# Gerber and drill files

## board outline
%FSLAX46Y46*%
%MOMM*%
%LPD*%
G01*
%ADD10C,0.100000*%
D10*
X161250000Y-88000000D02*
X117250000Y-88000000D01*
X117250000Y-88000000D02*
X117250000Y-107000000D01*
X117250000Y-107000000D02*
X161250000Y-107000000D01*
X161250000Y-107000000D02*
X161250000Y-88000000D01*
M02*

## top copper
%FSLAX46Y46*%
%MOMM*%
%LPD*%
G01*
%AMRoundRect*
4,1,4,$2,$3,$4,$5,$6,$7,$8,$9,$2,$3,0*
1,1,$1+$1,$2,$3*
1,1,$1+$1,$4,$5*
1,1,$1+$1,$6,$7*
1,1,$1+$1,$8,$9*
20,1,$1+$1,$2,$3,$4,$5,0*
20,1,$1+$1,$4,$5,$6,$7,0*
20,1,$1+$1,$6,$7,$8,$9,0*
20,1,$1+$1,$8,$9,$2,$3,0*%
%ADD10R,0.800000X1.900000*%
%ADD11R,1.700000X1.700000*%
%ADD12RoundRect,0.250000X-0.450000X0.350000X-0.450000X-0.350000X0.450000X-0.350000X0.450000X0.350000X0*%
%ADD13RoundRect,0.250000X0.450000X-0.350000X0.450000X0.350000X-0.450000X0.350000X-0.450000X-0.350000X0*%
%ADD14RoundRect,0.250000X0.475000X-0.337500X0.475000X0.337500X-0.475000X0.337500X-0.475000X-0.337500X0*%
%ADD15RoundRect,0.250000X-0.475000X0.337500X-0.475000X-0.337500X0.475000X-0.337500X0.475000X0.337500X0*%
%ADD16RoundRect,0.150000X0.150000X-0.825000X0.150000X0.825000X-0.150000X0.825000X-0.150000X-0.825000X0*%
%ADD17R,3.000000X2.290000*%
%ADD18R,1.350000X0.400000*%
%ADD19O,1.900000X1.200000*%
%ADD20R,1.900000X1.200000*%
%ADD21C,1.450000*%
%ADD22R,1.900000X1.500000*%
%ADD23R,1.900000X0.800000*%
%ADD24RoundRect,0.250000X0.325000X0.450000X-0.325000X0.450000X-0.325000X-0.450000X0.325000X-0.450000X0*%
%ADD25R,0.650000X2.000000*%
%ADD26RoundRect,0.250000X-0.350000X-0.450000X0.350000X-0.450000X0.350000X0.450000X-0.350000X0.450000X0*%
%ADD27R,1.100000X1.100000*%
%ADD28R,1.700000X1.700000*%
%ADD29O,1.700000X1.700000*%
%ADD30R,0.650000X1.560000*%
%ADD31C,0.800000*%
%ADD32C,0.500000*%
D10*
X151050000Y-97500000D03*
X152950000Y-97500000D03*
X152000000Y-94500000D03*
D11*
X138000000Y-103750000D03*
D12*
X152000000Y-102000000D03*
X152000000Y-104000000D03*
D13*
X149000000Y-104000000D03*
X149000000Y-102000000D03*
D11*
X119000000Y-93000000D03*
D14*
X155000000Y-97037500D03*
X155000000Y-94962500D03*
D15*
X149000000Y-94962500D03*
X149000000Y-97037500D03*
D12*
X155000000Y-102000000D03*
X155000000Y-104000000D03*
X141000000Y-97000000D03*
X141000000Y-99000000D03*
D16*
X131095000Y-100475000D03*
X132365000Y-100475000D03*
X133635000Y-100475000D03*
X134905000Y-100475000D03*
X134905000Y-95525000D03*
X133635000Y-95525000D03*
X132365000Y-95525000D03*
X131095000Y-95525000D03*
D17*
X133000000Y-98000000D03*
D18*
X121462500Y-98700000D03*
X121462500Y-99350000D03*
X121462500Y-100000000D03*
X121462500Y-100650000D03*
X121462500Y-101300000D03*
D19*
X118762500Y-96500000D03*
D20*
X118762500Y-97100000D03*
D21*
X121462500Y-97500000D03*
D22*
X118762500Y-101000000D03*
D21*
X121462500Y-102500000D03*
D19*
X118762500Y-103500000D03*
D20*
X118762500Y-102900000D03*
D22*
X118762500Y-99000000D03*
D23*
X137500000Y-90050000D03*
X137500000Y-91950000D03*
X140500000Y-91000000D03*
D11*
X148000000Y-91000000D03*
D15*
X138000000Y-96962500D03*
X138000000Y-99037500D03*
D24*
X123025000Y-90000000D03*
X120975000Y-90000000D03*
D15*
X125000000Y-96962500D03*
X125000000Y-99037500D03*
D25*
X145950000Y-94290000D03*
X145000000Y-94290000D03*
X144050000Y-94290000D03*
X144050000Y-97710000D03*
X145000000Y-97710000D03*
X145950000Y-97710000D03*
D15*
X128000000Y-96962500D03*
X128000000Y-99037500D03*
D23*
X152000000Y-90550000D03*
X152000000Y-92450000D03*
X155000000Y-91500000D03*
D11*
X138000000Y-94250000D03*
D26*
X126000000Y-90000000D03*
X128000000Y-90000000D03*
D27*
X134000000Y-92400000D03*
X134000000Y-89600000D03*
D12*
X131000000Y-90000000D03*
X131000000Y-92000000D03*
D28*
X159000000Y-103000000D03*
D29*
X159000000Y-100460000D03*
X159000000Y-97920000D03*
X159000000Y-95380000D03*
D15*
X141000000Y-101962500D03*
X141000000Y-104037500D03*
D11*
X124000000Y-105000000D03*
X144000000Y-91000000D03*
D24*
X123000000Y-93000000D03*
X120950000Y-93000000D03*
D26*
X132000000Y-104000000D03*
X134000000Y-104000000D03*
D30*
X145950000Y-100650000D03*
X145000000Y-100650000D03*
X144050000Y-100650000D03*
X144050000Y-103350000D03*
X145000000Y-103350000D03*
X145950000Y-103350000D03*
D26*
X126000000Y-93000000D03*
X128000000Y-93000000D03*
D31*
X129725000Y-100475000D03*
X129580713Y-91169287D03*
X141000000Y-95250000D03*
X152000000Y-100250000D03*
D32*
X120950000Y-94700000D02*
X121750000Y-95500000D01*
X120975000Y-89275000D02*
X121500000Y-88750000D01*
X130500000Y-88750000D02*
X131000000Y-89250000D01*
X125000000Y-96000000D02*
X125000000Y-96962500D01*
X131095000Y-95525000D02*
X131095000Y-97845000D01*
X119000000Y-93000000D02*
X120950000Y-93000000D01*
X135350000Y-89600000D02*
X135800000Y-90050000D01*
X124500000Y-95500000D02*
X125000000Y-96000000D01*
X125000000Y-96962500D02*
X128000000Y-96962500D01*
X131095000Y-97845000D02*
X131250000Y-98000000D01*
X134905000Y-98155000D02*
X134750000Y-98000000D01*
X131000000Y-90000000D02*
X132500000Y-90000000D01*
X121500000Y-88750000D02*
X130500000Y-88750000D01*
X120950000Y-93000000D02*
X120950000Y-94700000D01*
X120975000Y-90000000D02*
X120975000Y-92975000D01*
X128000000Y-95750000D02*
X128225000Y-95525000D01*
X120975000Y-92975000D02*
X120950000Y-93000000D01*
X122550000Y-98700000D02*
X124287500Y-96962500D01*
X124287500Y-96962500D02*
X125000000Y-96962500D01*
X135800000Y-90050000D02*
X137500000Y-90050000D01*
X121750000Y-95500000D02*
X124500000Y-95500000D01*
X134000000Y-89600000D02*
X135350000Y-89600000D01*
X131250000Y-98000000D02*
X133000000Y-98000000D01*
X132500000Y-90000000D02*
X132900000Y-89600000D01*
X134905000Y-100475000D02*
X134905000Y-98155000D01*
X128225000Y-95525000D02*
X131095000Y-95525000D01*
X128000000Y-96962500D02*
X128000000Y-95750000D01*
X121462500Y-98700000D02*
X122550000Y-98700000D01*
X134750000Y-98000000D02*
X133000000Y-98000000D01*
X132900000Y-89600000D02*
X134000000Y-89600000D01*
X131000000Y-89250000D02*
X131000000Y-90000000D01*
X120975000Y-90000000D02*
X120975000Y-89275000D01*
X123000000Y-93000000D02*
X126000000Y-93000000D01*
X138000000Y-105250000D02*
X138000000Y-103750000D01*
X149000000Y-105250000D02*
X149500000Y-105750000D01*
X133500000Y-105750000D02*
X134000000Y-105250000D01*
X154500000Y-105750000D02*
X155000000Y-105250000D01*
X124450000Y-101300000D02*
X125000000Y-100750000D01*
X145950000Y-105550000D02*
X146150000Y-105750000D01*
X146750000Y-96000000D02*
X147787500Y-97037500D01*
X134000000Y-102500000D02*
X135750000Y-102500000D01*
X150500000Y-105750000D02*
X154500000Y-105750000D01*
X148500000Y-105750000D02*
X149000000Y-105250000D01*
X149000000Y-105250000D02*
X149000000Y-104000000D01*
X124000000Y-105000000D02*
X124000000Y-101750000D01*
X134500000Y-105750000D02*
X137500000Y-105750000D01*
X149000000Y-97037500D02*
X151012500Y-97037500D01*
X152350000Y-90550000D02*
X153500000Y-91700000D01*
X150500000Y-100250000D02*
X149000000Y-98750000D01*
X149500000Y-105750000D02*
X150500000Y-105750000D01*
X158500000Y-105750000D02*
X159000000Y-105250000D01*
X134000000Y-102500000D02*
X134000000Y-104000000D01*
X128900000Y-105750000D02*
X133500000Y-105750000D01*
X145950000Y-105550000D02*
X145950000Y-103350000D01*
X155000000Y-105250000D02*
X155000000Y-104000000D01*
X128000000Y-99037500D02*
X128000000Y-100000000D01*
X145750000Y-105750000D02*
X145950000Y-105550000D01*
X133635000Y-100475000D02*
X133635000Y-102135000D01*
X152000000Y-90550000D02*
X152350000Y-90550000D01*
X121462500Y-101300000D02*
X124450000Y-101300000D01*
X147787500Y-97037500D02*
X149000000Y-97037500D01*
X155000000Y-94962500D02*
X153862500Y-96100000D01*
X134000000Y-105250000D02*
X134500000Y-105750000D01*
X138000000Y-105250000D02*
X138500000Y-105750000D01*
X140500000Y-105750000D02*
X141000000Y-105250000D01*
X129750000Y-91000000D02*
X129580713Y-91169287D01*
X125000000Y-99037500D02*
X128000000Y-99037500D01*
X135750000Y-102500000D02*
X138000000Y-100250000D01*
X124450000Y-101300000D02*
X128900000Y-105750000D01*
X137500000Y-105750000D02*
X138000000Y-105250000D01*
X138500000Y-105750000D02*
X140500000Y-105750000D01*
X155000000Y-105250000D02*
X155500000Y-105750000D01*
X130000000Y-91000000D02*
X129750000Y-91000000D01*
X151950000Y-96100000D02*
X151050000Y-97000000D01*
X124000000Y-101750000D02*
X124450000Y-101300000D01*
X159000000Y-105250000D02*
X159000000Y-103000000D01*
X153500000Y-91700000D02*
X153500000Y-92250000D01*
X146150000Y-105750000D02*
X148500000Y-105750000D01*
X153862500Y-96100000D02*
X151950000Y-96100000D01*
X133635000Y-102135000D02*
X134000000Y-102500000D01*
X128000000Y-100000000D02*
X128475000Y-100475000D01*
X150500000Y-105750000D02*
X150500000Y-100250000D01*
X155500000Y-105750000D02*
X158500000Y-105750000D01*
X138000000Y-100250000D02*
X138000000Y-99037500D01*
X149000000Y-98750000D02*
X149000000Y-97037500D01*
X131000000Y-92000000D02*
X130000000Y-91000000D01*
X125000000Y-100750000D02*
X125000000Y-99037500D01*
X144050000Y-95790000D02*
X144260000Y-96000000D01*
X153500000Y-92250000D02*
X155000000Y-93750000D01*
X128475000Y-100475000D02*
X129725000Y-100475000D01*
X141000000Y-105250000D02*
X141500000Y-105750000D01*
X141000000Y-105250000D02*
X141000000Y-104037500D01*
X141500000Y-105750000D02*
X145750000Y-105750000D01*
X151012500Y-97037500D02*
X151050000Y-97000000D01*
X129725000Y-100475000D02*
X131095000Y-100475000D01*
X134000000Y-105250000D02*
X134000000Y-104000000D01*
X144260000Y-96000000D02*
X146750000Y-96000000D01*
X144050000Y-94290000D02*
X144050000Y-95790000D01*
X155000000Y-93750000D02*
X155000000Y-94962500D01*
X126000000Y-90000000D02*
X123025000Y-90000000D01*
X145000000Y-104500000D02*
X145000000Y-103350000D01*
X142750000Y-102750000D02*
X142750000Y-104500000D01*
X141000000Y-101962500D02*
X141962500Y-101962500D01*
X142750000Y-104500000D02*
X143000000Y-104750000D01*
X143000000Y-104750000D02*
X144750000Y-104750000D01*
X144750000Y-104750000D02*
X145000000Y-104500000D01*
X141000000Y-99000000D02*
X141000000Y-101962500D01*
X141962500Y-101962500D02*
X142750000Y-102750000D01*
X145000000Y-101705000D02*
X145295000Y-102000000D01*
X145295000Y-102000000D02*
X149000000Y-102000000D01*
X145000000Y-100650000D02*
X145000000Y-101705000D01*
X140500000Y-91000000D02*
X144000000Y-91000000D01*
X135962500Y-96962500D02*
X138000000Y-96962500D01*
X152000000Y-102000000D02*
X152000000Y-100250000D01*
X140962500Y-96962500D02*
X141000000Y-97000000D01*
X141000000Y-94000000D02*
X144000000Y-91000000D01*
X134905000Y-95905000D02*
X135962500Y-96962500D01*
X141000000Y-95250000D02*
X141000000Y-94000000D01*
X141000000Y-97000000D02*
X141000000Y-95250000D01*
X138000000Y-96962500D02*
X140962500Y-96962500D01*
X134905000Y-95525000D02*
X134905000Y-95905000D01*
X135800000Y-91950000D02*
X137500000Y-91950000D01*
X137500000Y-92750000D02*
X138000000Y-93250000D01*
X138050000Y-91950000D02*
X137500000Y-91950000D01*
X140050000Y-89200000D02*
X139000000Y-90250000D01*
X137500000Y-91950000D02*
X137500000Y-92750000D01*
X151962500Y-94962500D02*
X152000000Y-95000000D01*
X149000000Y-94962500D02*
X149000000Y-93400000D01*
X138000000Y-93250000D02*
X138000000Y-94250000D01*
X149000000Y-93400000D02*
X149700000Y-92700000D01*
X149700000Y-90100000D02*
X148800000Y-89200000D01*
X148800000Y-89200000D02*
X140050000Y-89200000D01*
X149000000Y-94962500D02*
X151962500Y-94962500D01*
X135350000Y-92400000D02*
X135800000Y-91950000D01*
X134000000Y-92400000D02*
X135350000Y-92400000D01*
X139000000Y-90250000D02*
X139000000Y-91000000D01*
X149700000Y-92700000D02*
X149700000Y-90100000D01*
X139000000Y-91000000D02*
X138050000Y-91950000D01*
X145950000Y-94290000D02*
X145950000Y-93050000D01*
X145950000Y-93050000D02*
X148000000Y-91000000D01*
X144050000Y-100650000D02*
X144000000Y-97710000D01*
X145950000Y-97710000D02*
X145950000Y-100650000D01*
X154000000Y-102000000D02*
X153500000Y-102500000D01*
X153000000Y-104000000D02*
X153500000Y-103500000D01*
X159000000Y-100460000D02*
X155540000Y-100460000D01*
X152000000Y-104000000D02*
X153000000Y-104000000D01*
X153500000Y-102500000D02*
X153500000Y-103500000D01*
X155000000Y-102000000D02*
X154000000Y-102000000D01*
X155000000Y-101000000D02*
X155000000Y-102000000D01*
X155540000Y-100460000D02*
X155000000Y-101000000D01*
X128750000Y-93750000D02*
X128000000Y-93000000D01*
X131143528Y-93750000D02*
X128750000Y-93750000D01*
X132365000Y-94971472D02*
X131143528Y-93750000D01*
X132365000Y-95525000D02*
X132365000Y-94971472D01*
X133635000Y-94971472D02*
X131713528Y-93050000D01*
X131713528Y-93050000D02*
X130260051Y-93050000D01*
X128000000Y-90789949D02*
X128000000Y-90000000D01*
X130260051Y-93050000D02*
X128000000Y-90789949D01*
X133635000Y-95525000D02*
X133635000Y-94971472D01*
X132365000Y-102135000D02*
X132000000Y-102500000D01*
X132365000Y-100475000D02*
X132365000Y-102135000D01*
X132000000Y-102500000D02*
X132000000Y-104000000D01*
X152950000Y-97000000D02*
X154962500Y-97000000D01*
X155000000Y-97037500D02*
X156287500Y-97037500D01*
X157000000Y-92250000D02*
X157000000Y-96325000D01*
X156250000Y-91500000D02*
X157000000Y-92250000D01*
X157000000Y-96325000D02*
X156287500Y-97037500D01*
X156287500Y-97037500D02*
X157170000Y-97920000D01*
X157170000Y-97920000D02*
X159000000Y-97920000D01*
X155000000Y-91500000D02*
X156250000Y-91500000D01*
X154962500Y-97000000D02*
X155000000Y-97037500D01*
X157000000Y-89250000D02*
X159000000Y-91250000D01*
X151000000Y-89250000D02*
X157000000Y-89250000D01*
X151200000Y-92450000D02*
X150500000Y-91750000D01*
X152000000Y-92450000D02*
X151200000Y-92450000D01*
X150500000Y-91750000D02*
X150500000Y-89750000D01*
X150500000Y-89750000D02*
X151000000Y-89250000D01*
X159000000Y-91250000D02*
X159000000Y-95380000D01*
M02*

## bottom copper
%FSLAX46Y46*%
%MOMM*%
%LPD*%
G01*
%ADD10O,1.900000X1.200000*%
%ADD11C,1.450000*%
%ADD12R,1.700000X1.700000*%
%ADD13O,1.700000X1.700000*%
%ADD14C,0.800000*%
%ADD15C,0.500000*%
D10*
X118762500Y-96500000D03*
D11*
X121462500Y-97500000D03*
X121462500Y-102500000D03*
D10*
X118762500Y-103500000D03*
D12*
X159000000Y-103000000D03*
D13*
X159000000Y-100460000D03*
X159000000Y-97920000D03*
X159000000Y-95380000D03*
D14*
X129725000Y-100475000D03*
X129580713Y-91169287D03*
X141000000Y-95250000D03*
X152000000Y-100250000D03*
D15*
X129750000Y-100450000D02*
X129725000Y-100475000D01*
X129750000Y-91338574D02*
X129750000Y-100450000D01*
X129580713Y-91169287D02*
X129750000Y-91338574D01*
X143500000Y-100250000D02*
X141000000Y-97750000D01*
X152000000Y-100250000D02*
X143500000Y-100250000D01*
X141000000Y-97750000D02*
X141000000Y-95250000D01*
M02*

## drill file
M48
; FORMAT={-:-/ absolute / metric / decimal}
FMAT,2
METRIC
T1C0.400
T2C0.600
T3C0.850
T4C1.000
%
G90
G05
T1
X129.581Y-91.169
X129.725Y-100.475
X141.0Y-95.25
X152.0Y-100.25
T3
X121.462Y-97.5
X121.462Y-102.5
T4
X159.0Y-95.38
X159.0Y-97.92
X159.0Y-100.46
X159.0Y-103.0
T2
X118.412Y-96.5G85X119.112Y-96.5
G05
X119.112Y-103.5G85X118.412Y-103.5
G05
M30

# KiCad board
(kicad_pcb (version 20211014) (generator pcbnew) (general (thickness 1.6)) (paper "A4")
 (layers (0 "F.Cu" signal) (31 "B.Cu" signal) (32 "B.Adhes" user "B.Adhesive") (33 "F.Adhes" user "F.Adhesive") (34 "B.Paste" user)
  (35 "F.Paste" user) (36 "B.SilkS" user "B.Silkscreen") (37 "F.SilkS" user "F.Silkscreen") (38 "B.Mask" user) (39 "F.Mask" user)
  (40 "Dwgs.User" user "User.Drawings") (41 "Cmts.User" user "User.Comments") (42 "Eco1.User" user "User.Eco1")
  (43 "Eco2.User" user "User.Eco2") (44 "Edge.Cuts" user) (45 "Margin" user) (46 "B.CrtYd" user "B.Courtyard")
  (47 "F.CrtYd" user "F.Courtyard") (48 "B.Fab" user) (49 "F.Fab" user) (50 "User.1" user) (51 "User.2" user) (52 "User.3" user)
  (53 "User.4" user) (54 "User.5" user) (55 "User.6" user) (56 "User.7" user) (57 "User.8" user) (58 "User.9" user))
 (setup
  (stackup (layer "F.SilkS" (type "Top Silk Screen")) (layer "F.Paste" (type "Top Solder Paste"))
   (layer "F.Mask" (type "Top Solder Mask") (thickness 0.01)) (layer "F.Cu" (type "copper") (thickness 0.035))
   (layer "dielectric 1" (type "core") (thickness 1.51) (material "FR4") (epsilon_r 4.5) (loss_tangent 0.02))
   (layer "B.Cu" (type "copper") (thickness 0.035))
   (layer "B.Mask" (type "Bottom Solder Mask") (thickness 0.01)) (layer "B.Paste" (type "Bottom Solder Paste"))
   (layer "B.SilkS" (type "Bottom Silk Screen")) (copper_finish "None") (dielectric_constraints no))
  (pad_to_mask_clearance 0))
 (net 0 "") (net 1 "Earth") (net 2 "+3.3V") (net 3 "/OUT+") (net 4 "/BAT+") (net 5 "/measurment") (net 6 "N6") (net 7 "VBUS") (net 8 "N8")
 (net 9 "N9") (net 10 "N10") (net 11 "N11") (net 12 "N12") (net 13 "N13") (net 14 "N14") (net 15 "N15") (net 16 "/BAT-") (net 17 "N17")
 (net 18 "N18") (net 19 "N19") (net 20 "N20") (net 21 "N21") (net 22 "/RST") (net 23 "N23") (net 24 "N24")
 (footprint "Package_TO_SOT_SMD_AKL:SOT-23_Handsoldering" (layer "F.Cu") (at 152 96 90)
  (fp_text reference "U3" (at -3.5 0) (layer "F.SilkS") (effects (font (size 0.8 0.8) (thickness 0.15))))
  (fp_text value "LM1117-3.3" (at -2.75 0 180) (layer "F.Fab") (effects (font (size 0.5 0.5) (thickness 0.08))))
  (pad "1" smd rect (at -1.5 -0.95 90) (size 1.9 0.8) (layers "F.Cu" "F.Paste" "F.Mask") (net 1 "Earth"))
  (pad "2" smd rect (at -1.5 0.95 90) (size 1.9 0.8) (layers "F.Cu" "F.Paste" "F.Mask") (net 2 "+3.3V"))
  (pad "3" smd rect (at 1.5 0 90) (size 1.9 0.8) (layers "F.Cu" "F.Paste" "F.Mask") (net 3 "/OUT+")))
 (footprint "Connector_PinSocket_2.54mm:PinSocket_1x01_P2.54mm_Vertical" (layer "F.Cu") (at 138 103.75)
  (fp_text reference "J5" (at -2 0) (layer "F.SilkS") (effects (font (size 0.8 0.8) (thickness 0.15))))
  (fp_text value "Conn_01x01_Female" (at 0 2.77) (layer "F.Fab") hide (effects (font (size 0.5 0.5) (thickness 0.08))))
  (pad "1" smd rect (at 0 0) (size 1.7 1.7) (layers "F.Cu" "F.Paste" "F.Mask") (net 1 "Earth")))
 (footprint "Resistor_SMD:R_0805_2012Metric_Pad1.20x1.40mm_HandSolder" (layer "F.Cu") (at 152 103 -90)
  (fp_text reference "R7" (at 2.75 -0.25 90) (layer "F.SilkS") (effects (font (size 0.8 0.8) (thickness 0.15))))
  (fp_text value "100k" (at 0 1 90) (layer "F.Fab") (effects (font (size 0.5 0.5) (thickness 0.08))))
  (pad "1" smd roundrect (at -1 0 270) (size 1.2 1.4) (layers "F.Cu" "F.Paste" "F.Mask") (roundrect_rratio 0.2083333333) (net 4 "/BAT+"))
  (pad "2" smd roundrect (at 1 0 270) (size 1.2 1.4) (layers "F.Cu" "F.Paste" "F.Mask") (roundrect_rratio 0.2083333333)
   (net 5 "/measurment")))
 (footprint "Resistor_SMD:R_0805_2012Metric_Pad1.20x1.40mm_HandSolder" (layer "F.Cu") (at 149 103 90)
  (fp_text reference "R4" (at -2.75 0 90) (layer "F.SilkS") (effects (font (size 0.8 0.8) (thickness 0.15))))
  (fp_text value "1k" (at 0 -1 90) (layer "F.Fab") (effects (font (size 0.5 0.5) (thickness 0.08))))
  (pad "1" smd roundrect (at -1 0 90) (size 1.2 1.4) (layers "F.Cu" "F.Paste" "F.Mask") (roundrect_rratio 0.2083333333) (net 1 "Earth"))
  (pad "2" smd roundrect (at 1 0 90) (size 1.2 1.4) (layers "F.Cu" "F.Paste" "F.Mask") (roundrect_rratio 0.2083333333) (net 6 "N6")))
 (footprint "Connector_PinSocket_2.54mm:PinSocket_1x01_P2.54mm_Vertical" (layer "F.Cu") (at 119 93)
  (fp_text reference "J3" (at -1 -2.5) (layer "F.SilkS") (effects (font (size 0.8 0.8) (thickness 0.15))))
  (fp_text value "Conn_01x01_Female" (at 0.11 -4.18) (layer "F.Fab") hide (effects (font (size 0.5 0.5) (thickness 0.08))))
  (pad "1" smd rect (at 0 0) (size 1.7 1.7) (layers "F.Cu" "F.Paste" "F.Mask") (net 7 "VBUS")))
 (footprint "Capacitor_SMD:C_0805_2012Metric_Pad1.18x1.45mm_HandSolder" (layer "F.Cu") (at 155 96 90)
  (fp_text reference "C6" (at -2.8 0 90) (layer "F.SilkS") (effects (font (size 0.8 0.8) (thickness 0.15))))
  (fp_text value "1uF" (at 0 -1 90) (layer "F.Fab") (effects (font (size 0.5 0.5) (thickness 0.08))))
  (pad "1" smd roundrect (at -1.0375 0 90) (size 1.175 1.45) (layers "F.Cu" "F.Paste" "F.Mask") (roundrect_rratio 0.2127659574)
   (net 2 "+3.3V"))
  (pad "2" smd roundrect (at 1.0375 0 90) (size 1.175 1.45) (layers "F.Cu" "F.Paste" "F.Mask") (roundrect_rratio 0.2127659574)
   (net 1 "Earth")))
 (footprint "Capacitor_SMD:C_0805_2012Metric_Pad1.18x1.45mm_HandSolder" (layer "F.Cu") (at 149 96 -90)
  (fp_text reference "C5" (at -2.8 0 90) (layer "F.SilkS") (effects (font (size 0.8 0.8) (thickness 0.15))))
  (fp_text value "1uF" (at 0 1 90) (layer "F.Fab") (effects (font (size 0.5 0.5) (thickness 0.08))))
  (pad "1" smd roundrect (at -1.0375 0 270) (size 1.175 1.45) (layers "F.Cu" "F.Paste" "F.Mask") (roundrect_rratio 0.2127659574)
   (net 3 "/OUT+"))
  (pad "2" smd roundrect (at 1.0375 0 270) (size 1.175 1.45) (layers "F.Cu" "F.Paste" "F.Mask") (roundrect_rratio 0.2127659574)
   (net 1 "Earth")))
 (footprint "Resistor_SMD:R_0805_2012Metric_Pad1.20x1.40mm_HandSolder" (layer "F.Cu") (at 155 103 -90)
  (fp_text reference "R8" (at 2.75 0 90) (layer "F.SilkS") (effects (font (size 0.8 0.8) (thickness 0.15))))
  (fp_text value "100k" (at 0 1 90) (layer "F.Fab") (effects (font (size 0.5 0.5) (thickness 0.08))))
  (pad "1" smd roundrect (at -1 0 270) (size 1.2 1.4) (layers "F.Cu" "F.Paste" "F.Mask") (roundrect_rratio 0.2083333333)
   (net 5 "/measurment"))
  (pad "2" smd roundrect (at 1 0 270) (size 1.2 1.4) (layers "F.Cu" "F.Paste" "F.Mask") (roundrect_rratio 0.2083333333) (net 1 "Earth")))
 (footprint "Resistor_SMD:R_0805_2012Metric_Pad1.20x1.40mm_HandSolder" (layer "F.Cu") (at 141 98 -90)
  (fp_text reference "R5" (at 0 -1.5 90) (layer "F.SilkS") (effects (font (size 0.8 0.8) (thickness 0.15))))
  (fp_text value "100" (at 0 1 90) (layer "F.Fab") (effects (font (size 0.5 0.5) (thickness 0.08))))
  (pad "1" smd roundrect (at -1 0 270) (size 1.2 1.4) (layers "F.Cu" "F.Paste" "F.Mask") (roundrect_rratio 0.2083333333) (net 4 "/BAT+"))
  (pad "2" smd roundrect (at 1 0 270) (size 1.2 1.4) (layers "F.Cu" "F.Paste" "F.Mask") (roundrect_rratio 0.2083333333) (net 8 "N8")))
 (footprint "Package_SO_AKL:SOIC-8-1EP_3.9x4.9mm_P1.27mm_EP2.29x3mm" (layer "F.Cu") (at 133 98 90)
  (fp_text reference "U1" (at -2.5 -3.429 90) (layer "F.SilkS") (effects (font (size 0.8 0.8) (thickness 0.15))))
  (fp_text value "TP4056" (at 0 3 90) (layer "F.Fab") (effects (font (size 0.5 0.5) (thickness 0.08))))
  (pad "" smd roundrect (at 0.57 -0.75 90) (size 0.92 1.21) (layers "F.Paste") (roundrect_rratio 0.25))
  (pad "" smd roundrect (at -0.57 0.75 90) (size 0.92 1.21) (layers "F.Paste") (roundrect_rratio 0.25))
  (pad "" smd roundrect (at 0.57 0.75 90) (size 0.92 1.21) (layers "F.Paste") (roundrect_rratio 0.25))
  (pad "" smd roundrect (at -0.57 -0.75 90) (size 0.92 1.21) (layers "F.Paste") (roundrect_rratio 0.25))
  (pad "1" smd roundrect (at -2.475 -1.905 90) (size 1.95 0.6) (layers "F.Cu" "F.Paste" "F.Mask") (roundrect_rratio 0.25) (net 1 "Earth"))
  (pad "2" smd roundrect (at -2.475 -0.635 90) (size 1.95 0.6) (layers "F.Cu" "F.Paste" "F.Mask") (roundrect_rratio 0.25) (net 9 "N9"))
  (pad "3" smd roundrect (at -2.475 0.635 90) (size 1.95 0.6) (layers "F.Cu" "F.Paste" "F.Mask") (roundrect_rratio 0.25) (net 1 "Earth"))
  (pad "4" smd roundrect (at -2.475 1.905 90) (size 1.95 0.6) (layers "F.Cu" "F.Paste" "F.Mask") (roundrect_rratio 0.25) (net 7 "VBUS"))
  (pad "5" smd roundrect (at 2.475 1.905 90) (size 1.95 0.6) (layers "F.Cu" "F.Paste" "F.Mask") (roundrect_rratio 0.25) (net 4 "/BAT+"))
  (pad "6" smd roundrect (at 2.475 0.635 90) (size 1.95 0.6) (layers "F.Cu" "F.Paste" "F.Mask") (roundrect_rratio 0.25) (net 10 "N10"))
  (pad "7" smd roundrect (at 2.475 -0.635 90) (size 1.95 0.6) (layers "F.Cu" "F.Paste" "F.Mask") (roundrect_rratio 0.25) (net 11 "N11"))
  (pad "8" smd roundrect (at 2.475 -1.905 90) (size 1.95 0.6) (layers "F.Cu" "F.Paste" "F.Mask") (roundrect_rratio 0.25) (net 7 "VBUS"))
  (pad "9" smd rect (at 0 0 90) (size 2.29 3) (layers "F.Cu" "F.Mask") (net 7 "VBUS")))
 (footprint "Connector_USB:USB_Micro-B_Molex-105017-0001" (layer "F.Cu") (at 120 100 -90)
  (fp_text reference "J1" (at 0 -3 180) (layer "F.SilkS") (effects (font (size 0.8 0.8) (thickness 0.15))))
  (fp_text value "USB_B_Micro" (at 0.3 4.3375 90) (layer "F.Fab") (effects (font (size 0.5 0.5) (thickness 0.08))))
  (pad "1" smd rect (at -1.3 -1.4625 270) (size 0.4 1.35) (layers "F.Cu" "F.Paste" "F.Mask") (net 7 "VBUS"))
  (pad "2" smd rect (at -0.65 -1.4625 270) (size 0.4 1.35) (layers "F.Cu" "F.Paste" "F.Mask") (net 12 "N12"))
  (pad "3" smd rect (at 0 -1.4625 270) (size 0.4 1.35) (layers "F.Cu" "F.Paste" "F.Mask") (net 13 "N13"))
  (pad "4" smd rect (at 0.65 -1.4625 270) (size 0.4 1.35) (layers "F.Cu" "F.Paste" "F.Mask") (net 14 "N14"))
  (pad "5" smd rect (at 1.3 -1.4625 270) (size 0.4 1.35) (layers "F.Cu" "F.Paste" "F.Mask") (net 1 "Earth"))
  (pad "6" thru_hole oval (at -3.5 1.2375 90) (size 1.2 1.9) (drill oval 0.6 1.3) (layers *.Cu *.Mask) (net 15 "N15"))
  (pad "6" smd rect (at -2.9 1.2375 270) (size 1.2 1.9) (layers "F.Cu" "F.Mask") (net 15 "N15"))
  (pad "6" thru_hole circle (at -2.5 -1.4625 270) (size 1.45 1.45) (drill 0.85) (layers *.Cu *.Mask) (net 15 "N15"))
  (pad "6" smd rect (at 1 1.2375 270) (size 1.5 1.9) (layers "F.Cu" "F.Paste" "F.Mask") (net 15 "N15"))
  (pad "6" thru_hole circle (at 2.5 -1.4625 270) (size 1.45 1.45) (drill 0.85) (layers *.Cu *.Mask) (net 15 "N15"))
  (pad "6" thru_hole oval (at 3.5 1.2375 270) (size 1.2 1.9) (drill oval 0.6 1.3) (layers *.Cu *.Mask) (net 15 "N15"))
  (pad "6" smd rect (at 2.9 1.2375 270) (size 1.2 1.9) (layers "F.Cu" "F.Mask") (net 15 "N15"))
  (pad "6" smd rect (at -1 1.2375 270) (size 1.5 1.9) (layers "F.Cu" "F.Paste" "F.Mask") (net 15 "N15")))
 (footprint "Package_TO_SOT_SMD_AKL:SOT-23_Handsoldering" (layer "F.Cu") (at 139 91)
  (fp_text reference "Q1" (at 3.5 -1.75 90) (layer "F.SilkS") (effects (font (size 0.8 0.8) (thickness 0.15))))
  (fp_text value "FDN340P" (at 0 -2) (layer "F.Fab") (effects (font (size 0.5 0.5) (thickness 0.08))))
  (pad "1" smd rect (at -1.5 -0.95) (size 1.9 0.8) (layers "F.Cu" "F.Paste" "F.Mask") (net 7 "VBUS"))
  (pad "2" smd rect (at -1.5 0.95) (size 1.9 0.8) (layers "F.Cu" "F.Paste" "F.Mask") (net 3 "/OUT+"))
  (pad "3" smd rect (at 1.5 0) (size 1.9 0.8) (layers "F.Cu" "F.Paste" "F.Mask") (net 4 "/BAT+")))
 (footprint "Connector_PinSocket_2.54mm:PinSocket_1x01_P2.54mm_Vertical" (layer "F.Cu") (at 148 91)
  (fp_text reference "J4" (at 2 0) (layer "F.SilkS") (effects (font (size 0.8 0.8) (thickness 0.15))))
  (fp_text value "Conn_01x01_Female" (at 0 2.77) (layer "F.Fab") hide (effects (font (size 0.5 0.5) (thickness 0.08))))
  (pad "1" smd rect (at 0 0) (size 1.7 1.7) (layers "F.Cu" "F.Paste" "F.Mask") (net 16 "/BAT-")))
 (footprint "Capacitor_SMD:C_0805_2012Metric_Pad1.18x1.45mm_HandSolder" (layer "F.Cu") (at 138 98 -90)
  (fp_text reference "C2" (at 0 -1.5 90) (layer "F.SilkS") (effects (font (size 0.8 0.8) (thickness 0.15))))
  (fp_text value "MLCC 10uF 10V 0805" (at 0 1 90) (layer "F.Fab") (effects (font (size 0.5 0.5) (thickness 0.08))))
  (pad "1" smd roundrect (at -1.0375 0 270) (size 1.175 1.45) (layers "F.Cu" "F.Paste" "F.Mask") (roundrect_rratio 0.2127659574)
   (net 4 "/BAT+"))
  (pad "2" smd roundrect (at 1.0375 0 270) (size 1.175 1.45) (layers "F.Cu" "F.Paste" "F.Mask") (roundrect_rratio 0.2127659574)
   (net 1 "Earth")))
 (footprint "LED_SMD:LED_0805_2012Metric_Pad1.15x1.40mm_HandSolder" (layer "F.Cu") (at 122 90 180)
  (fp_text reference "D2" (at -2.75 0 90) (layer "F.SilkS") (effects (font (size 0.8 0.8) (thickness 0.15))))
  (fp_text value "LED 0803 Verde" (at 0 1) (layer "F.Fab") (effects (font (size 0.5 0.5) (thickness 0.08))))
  (pad "1" smd roundrect (at -1.025 0 180) (size 1.15 1.4) (layers "F.Cu" "F.Paste" "F.Mask") (roundrect_rratio 0.2173913043) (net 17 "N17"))
  (pad "2" smd roundrect (at 1.025 0 180) (size 1.15 1.4) (layers "F.Cu" "F.Paste" "F.Mask") (roundrect_rratio 0.2173913043) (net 7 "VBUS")))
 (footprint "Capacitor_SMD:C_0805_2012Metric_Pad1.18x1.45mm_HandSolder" (layer "F.Cu") (at 125 98 -90)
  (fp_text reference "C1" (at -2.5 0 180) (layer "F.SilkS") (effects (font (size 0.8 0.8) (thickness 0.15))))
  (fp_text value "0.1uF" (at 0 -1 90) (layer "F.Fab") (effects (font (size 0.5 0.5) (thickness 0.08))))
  (pad "1" smd roundrect (at -1.0375 0 270) (size 1.175 1.45) (layers "F.Cu" "F.Paste" "F.Mask") (roundrect_rratio 0.2127659574)
   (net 7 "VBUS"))
  (pad "2" smd roundrect (at 1.0375 0 270) (size 1.175 1.45) (layers "F.Cu" "F.Paste" "F.Mask") (roundrect_rratio 0.2127659574)
   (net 1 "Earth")))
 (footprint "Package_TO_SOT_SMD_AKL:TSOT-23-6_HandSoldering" (layer "F.Cu") (at 145 96 -90)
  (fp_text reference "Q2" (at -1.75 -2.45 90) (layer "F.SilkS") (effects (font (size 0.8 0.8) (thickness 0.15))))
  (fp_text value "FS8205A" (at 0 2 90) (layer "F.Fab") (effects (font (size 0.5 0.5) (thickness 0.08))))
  (pad "1" smd rect (at -1.71 -0.95 270) (size 2 0.65) (layers "F.Cu" "F.Paste" "F.Mask") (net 16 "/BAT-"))
  (pad "2" smd rect (at -1.71 0 270) (size 2 0.65) (layers "F.Cu" "F.Paste" "F.Mask") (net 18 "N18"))
  (pad "3" smd rect (at -1.71 0.95 270) (size 2 0.65) (layers "F.Cu" "F.Paste" "F.Mask") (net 1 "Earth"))
  (pad "4" smd rect (at 1.71 0.95 270) (size 2 0.65) (layers "F.Cu" "F.Paste" "F.Mask") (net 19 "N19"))
  (pad "5" smd rect (at 1.71 0 270) (size 2 0.65) (layers "F.Cu" "F.Paste" "F.Mask") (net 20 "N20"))
  (pad "6" smd rect (at 1.71 -0.95 270) (size 2 0.65) (layers "F.Cu" "F.Paste" "F.Mask") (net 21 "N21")))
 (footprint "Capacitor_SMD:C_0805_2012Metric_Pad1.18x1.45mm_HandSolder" (layer "F.Cu") (at 128 98 -90)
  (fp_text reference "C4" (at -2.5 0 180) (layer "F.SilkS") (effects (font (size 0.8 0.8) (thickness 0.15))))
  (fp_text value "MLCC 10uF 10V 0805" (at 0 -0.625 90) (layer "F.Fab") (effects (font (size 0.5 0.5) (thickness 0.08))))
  (pad "1" smd roundrect (at -1.0375 0 270) (size 1.175 1.45) (layers "F.Cu" "F.Paste" "F.Mask") (roundrect_rratio 0.2127659574)
   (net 7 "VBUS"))
  (pad "2" smd roundrect (at 1.0375 0 270) (size 1.175 1.45) (layers "F.Cu" "F.Paste" "F.Mask") (roundrect_rratio 0.2127659574)
   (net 1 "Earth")))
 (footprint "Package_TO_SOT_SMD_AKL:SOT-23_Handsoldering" (layer "F.Cu") (at 153.5 91.5)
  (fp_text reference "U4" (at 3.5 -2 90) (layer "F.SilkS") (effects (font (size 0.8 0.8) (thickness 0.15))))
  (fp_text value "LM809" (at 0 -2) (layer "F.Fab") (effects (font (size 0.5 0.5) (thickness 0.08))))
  (pad "1" smd rect (at -1.5 -0.95) (size 1.9 0.8) (layers "F.Cu" "F.Paste" "F.Mask") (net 1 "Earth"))
  (pad "2" smd rect (at -1.5 0.95) (size 1.9 0.8) (layers "F.Cu" "F.Paste" "F.Mask") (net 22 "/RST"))
  (pad "3" smd rect (at 1.5 0) (size 1.9 0.8) (layers "F.Cu" "F.Paste" "F.Mask") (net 2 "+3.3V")))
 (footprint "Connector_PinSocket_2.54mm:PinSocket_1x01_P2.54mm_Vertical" (layer "F.Cu") (at 138 94.25)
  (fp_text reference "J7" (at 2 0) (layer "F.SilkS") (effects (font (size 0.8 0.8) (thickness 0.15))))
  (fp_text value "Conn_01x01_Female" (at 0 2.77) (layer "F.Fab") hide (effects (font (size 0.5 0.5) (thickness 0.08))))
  (pad "1" smd rect (at 0 0) (size 1.7 1.7) (layers "F.Cu" "F.Paste" "F.Mask") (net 3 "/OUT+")))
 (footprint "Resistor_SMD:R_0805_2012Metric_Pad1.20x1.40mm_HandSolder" (layer "F.Cu") (at 127 90)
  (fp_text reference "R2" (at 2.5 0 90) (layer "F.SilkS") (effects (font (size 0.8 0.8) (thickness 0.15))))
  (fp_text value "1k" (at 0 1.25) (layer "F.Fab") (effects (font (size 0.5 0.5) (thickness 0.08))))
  (pad "1" smd roundrect (at -1 0) (size 1.2 1.4) (layers "F.Cu" "F.Paste" "F.Mask") (roundrect_rratio 0.2083333333) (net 17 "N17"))
  (pad "2" smd roundrect (at 1 0) (size 1.2 1.4) (layers "F.Cu" "F.Paste" "F.Mask") (roundrect_rratio 0.2083333333) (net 10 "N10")))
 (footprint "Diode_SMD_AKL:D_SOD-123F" (layer "F.Cu") (at 134 91 90)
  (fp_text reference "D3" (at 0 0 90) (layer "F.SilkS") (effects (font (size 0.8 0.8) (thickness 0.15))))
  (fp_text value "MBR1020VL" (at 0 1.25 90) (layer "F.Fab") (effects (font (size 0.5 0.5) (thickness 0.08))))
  (pad "1" smd rect (at -1.4 0 90) (size 1.1 1.1) (layers "F.Cu" "F.Paste" "F.Mask") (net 3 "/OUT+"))
  (pad "2" smd rect (at 1.4 0 90) (size 1.1 1.1) (layers "F.Cu" "F.Paste" "F.Mask") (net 7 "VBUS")))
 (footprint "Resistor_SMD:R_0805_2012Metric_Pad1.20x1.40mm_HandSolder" (layer "F.Cu") (at 131 91 -90)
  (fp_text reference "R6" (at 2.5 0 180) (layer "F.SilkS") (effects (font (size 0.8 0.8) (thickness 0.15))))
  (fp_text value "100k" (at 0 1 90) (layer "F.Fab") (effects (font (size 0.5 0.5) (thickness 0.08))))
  (pad "1" smd roundrect (at -1 0 270) (size 1.2 1.4) (layers "F.Cu" "F.Paste" "F.Mask") (roundrect_rratio 0.2083333333) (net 7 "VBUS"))
  (pad "2" smd roundrect (at 1 0 270) (size 1.2 1.4) (layers "F.Cu" "F.Paste" "F.Mask") (roundrect_rratio 0.2083333333) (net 1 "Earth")))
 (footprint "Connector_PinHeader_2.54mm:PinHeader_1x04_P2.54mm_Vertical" (layer "F.Cu") (at 159 103 180)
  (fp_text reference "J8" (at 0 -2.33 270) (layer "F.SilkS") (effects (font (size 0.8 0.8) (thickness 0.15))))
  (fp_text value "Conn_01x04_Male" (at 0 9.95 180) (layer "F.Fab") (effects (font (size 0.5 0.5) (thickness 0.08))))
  (pad "1" thru_hole rect (at 0 0 180) (size 1.7 1.7) (drill 1) (layers *.Cu *.Mask) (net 1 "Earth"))
  (pad "2" thru_hole oval (at 0 2.54 180) (size 1.7 1.7) (drill 1) (layers *.Cu *.Mask) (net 5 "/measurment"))
  (pad "3" thru_hole oval (at 0 5.08 180) (size 1.7 1.7) (drill 1) (layers *.Cu *.Mask) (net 2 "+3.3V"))
  (pad "4" thru_hole oval (at 0 7.62 180) (size 1.7 1.7) (drill 1) (layers *.Cu *.Mask) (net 22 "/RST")))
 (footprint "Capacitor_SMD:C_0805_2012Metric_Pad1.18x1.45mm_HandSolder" (layer "F.Cu") (at 141 103 -90)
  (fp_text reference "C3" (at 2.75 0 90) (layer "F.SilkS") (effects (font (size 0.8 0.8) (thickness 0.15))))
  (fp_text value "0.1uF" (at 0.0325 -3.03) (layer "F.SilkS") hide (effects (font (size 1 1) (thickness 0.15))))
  (pad "1" smd roundrect (at -1.0375 0 270) (size 1.175 1.45) (layers "F.Cu" "F.Paste" "F.Mask") (roundrect_rratio 0.2127659574)
   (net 8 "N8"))
  (pad "2" smd roundrect (at 1.0375 0 270) (size 1.175 1.45) (layers "F.Cu" "F.Paste" "F.Mask") (roundrect_rratio 0.2127659574)
   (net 1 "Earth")))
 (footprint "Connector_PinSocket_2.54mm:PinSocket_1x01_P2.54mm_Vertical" (layer "F.Cu") (at 124 105)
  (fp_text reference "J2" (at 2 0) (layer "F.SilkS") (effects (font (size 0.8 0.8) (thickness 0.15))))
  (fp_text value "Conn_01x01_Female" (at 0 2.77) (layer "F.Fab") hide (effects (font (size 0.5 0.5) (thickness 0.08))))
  (pad "1" smd rect (at 0 0) (size 1.7 1.7) (layers "F.Cu" "F.Paste" "F.Mask") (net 1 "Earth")))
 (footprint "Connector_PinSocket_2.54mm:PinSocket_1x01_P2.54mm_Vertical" (layer "F.Cu") (at 144 91)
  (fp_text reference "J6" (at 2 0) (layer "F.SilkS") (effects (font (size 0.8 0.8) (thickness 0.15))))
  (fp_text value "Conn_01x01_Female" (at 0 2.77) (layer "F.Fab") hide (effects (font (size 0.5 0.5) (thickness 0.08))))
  (pad "1" smd rect (at 0 0) (size 1.7 1.7) (layers "F.Cu" "F.Paste" "F.Mask") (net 4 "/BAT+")))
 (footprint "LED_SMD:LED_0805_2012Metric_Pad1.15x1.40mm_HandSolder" (layer "F.Cu") (at 121.975 93 180)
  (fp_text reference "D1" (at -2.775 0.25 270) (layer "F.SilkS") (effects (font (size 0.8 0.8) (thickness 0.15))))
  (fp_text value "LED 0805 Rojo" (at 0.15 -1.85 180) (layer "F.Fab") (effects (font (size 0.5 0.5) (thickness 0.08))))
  (pad "1" smd roundrect (at -1.025 0 180) (size 1.15 1.4) (layers "F.Cu" "F.Paste" "F.Mask") (roundrect_rratio 0.2173913043) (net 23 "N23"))
  (pad "2" smd roundrect (at 1.025 0 180) (size 1.15 1.4) (layers "F.Cu" "F.Paste" "F.Mask") (roundrect_rratio 0.2173913043) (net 7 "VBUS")))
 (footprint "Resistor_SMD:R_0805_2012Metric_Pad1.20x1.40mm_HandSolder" (layer "F.Cu") (at 133 104)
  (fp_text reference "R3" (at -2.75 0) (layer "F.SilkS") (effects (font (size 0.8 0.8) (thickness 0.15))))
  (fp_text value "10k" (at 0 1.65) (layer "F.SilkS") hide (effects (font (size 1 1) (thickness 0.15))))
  (pad "1" smd roundrect (at -1 0) (size 1.2 1.4) (layers "F.Cu" "F.Paste" "F.Mask") (roundrect_rratio 0.2083333333) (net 9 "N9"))
  (pad "2" smd roundrect (at 1 0) (size 1.2 1.4) (layers "F.Cu" "F.Paste" "F.Mask") (roundrect_rratio 0.2083333333) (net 1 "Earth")))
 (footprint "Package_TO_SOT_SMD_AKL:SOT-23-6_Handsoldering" (layer "F.Cu") (at 145 102 -90)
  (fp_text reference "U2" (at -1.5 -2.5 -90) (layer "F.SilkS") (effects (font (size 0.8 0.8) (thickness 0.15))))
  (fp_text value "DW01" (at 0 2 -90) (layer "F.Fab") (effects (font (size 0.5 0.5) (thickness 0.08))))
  (pad "1" smd rect (at -1.35 -0.95 270) (size 1.56 0.65) (layers "F.Cu" "F.Paste" "F.Mask") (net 21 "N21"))
  (pad "2" smd rect (at -1.35 0 270) (size 1.56 0.65) (layers "F.Cu" "F.Paste" "F.Mask") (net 6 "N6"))
  (pad "3" smd rect (at -1.35 0.95 270) (size 1.56 0.65) (layers "F.Cu" "F.Paste" "F.Mask") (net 19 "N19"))
  (pad "4" smd rect (at 1.35 0.95 270) (size 1.56 0.65) (layers "F.Cu" "F.Paste" "F.Mask") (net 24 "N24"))
  (pad "5" smd rect (at 1.35 0 270) (size 1.56 0.65) (layers "F.Cu" "F.Paste" "F.Mask") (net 8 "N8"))
  (pad "6" smd rect (at 1.35 -0.95 270) (size 1.56 0.65) (layers "F.Cu" "F.Paste" "F.Mask") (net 1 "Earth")))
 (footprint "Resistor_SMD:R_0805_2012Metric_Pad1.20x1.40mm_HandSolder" (layer "F.Cu") (at 127 93)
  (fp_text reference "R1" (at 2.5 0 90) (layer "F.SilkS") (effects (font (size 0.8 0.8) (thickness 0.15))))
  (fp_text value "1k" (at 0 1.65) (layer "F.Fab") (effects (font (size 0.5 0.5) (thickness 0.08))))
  (pad "1" smd roundrect (at -1 0) (size 1.2 1.4) (layers "F.Cu" "F.Paste" "F.Mask") (roundrect_rratio 0.2083333333) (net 23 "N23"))
  (pad "2" smd roundrect (at 1 0) (size 1.2 1.4) (layers "F.Cu" "F.Paste" "F.Mask") (roundrect_rratio 0.2083333333) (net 11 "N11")))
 (gr_line (start 161.25 88) (end 117.25 88) (layer "Edge.Cuts") (width 0.1))
 (gr_line (start 117.25 88) (end 117.25 107) (layer "Edge.Cuts") (width 0.1))
 (gr_line (start 117.25 107) (end 161.25 107) (layer "Edge.Cuts") (width 0.1))
 (gr_line (start 161.25 107) (end 161.25 88) (layer "Edge.Cuts") (width 0.1))
 (segment (start 120.95 94.7) (end 121.75 95.5) (width 0.5) (layer "F.Cu") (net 7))
 (segment (start 120.975 89.275) (end 121.5 88.75) (width 0.5) (layer "F.Cu") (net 7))
 (segment (start 130.5 88.75) (end 131 89.25) (width 0.5) (layer "F.Cu") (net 7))
 (segment (start 125 96) (end 125 96.9625) (width 0.5) (layer "F.Cu") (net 7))
 (segment (start 131.095 95.525) (end 131.095 97.845) (width 0.5) (layer "F.Cu") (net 7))
 (segment (start 119 93) (end 120.95 93) (width 0.5) (layer "F.Cu") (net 7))
 (segment (start 135.35 89.6) (end 135.8 90.05) (width 0.5) (layer "F.Cu") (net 7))
 (segment (start 124.5 95.5) (end 125 96) (width 0.5) (layer "F.Cu") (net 7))
 (segment (start 125 96.9625) (end 128 96.9625) (width 0.5) (layer "F.Cu") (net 7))
 (segment (start 131.095 97.845) (end 131.25 98) (width 0.5) (layer "F.Cu") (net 7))
 (segment (start 134.905 98.155) (end 134.75 98) (width 0.5) (layer "F.Cu") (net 7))
 (segment (start 131 90) (end 132.5 90) (width 0.5) (layer "F.Cu") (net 7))
 (segment (start 121.5 88.75) (end 130.5 88.75) (width 0.5) (layer "F.Cu") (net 7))
 (segment (start 120.95 93) (end 120.95 94.7) (width 0.5) (layer "F.Cu") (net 7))
 (segment (start 120.975 90) (end 120.975 92.975) (width 0.5) (layer "F.Cu") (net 7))
 (segment (start 128 95.75) (end 128.225 95.525) (width 0.5) (layer "F.Cu") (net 7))
 (segment (start 120.975 92.975) (end 120.95 93) (width 0.5) (layer "F.Cu") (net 7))
 (segment (start 122.55 98.7) (end 124.2875 96.9625) (width 0.5) (layer "F.Cu") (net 7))
 (segment (start 124.2875 96.9625) (end 125 96.9625) (width 0.5) (layer "F.Cu") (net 7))
 (segment (start 135.8 90.05) (end 137.5 90.05) (width 0.5) (layer "F.Cu") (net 7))
 (segment (start 121.75 95.5) (end 124.5 95.5) (width 0.5) (layer "F.Cu") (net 7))
 (segment (start 134 89.6) (end 135.35 89.6) (width 0.5) (layer "F.Cu") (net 7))
 (segment (start 131.25 98) (end 133 98) (width 0.5) (layer "F.Cu") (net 7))
 (segment (start 132.5 90) (end 132.9 89.6) (width 0.5) (layer "F.Cu") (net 7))
 (segment (start 134.905 100.475) (end 134.905 98.155) (width 0.5) (layer "F.Cu") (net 7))
 (segment (start 128.225 95.525) (end 131.095 95.525) (width 0.5) (layer "F.Cu") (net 7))
 (segment (start 128 96.9625) (end 128 95.75) (width 0.5) (layer "F.Cu") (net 7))
 (segment (start 121.4625 98.7) (end 122.55 98.7) (width 0.5) (layer "F.Cu") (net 7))
 (segment (start 134.75 98) (end 133 98) (width 0.5) (layer "F.Cu") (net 7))
 (segment (start 132.9 89.6) (end 134 89.6) (width 0.5) (layer "F.Cu") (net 7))
 (segment (start 131 89.25) (end 131 90) (width 0.5) (layer "F.Cu") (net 7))
 (segment (start 120.975 90) (end 120.975 89.275) (width 0.5) (layer "F.Cu") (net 7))
 (segment (start 123 93) (end 126 93) (width 0.5) (layer "F.Cu") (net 23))
 (segment (start 138 105.25) (end 138 103.75) (width 0.5) (layer "F.Cu") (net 1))
 (segment (start 149 105.25) (end 149.5 105.75) (width 0.5) (layer "F.Cu") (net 1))
 (segment (start 133.5 105.75) (end 134 105.25) (width 0.5) (layer "F.Cu") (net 1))
 (segment (start 154.5 105.75) (end 155 105.25) (width 0.5) (layer "F.Cu") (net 1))
 (segment (start 124.45 101.3) (end 125 100.75) (width 0.5) (layer "F.Cu") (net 1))
 (segment (start 145.95 105.55) (end 146.15 105.75) (width 0.5) (layer "F.Cu") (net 1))
 (segment (start 146.75 96) (end 147.7875 97.0375) (width 0.5) (layer "F.Cu") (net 1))
 (segment (start 134 102.5) (end 135.75 102.5) (width 0.5) (layer "F.Cu") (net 1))
 (segment (start 150.5 105.75) (end 154.5 105.75) (width 0.5) (layer "F.Cu") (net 1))
 (segment (start 148.5 105.75) (end 149 105.25) (width 0.5) (layer "F.Cu") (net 1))
 (segment (start 149 105.25) (end 149 104) (width 0.5) (layer "F.Cu") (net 1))
 (segment (start 124 105) (end 124 101.75) (width 0.5) (layer "F.Cu") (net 1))
 (segment (start 134.5 105.75) (end 137.5 105.75) (width 0.5) (layer "F.Cu") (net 1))
 (segment (start 149 97.0375) (end 151.0125 97.0375) (width 0.5) (layer "F.Cu") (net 1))
 (segment (start 152.35 90.55) (end 153.5 91.7) (width 0.5) (layer "F.Cu") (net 1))
 (segment (start 150.5 100.25) (end 149 98.75) (width 0.5) (layer "F.Cu") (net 1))
 (segment (start 149.5 105.75) (end 150.5 105.75) (width 0.5) (layer "F.Cu") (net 1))
 (segment (start 158.5 105.75) (end 159 105.25) (width 0.5) (layer "F.Cu") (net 1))
 (segment (start 134 102.5) (end 134 104) (width 0.5) (layer "F.Cu") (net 1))
 (segment (start 128.9 105.75) (end 133.5 105.75) (width 0.5) (layer "F.Cu") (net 1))
 (segment (start 145.95 105.55) (end 145.95 103.35) (width 0.5) (layer "F.Cu") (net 1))
 (segment (start 155 105.25) (end 155 104) (width 0.5) (layer "F.Cu") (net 1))
 (segment (start 128 99.0375) (end 128 100) (width 0.5) (layer "F.Cu") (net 1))
 (segment (start 145.75 105.75) (end 145.95 105.55) (width 0.5) (layer "F.Cu") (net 1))
 (segment (start 133.635 100.475) (end 133.635 102.135) (width 0.5) (layer "F.Cu") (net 1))
 (segment (start 152 90.55) (end 152.35 90.55) (width 0.5) (layer "F.Cu") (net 1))
 (segment (start 121.4625 101.3) (end 124.45 101.3) (width 0.5) (layer "F.Cu") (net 1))
 (segment (start 147.7875 97.0375) (end 149 97.0375) (width 0.5) (layer "F.Cu") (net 1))
 (segment (start 155 94.9625) (end 153.8625 96.1) (width 0.5) (layer "F.Cu") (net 1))
 (segment (start 134 105.25) (end 134.5 105.75) (width 0.5) (layer "F.Cu") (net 1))
 (segment (start 138 105.25) (end 138.5 105.75) (width 0.5) (layer "F.Cu") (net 1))
 (segment (start 140.5 105.75) (end 141 105.25) (width 0.5) (layer "F.Cu") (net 1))
 (segment (start 129.75 91) (end 129.580713 91.169287) (width 0.5) (layer "F.Cu") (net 1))
 (segment (start 125 99.0375) (end 128 99.0375) (width 0.5) (layer "F.Cu") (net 1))
 (segment (start 135.75 102.5) (end 138 100.25) (width 0.5) (layer "F.Cu") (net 1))
 (segment (start 124.45 101.3) (end 128.9 105.75) (width 0.5) (layer "F.Cu") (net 1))
 (segment (start 137.5 105.75) (end 138 105.25) (width 0.5) (layer "F.Cu") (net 1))
 (segment (start 138.5 105.75) (end 140.5 105.75) (width 0.5) (layer "F.Cu") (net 1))
 (segment (start 155 105.25) (end 155.5 105.75) (width 0.5) (layer "F.Cu") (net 1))
 (segment (start 130 91) (end 129.75 91) (width 0.5) (layer "F.Cu") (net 1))
 (segment (start 151.95 96.1) (end 151.05 97) (width 0.5) (layer "F.Cu") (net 1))
 (segment (start 124 101.75) (end 124.45 101.3) (width 0.5) (layer "F.Cu") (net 1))
 (segment (start 159 105.25) (end 159 103) (width 0.5) (layer "F.Cu") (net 1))
 (segment (start 153.5 91.7) (end 153.5 92.25) (width 0.5) (layer "F.Cu") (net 1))
 (segment (start 146.15 105.75) (end 148.5 105.75) (width 0.5) (layer "F.Cu") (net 1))
 (segment (start 153.8625 96.1) (end 151.95 96.1) (width 0.5) (layer "F.Cu") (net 1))
 (segment (start 133.635 102.135) (end 134 102.5) (width 0.5) (layer "F.Cu") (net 1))
 (segment (start 128 100) (end 128.475 100.475) (width 0.5) (layer "F.Cu") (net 1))
 (segment (start 150.5 105.75) (end 150.5 100.25) (width 0.5) (layer "F.Cu") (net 1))
 (segment (start 155.5 105.75) (end 158.5 105.75) (width 0.5) (layer "F.Cu") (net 1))
 (segment (start 138 100.25) (end 138 99.0375) (width 0.5) (layer "F.Cu") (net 1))
 (segment (start 149 98.75) (end 149 97.0375) (width 0.5) (layer "F.Cu") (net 1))
 (segment (start 131 92) (end 130 91) (width 0.5) (layer "F.Cu") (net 1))
 (segment (start 125 100.75) (end 125 99.0375) (width 0.5) (layer "F.Cu") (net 1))
 (segment (start 144.05 95.79) (end 144.26 96) (width 0.5) (layer "F.Cu") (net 1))
 (segment (start 153.5 92.25) (end 155 93.75) (width 0.5) (layer "F.Cu") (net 1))
 (segment (start 128.475 100.475) (end 129.725 100.475) (width 0.5) (layer "F.Cu") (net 1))
 (segment (start 141 105.25) (end 141.5 105.75) (width 0.5) (layer "F.Cu") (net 1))
 (segment (start 141 105.25) (end 141 104.0375) (width 0.5) (layer "F.Cu") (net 1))
 (segment (start 141.5 105.75) (end 145.75 105.75) (width 0.5) (layer "F.Cu") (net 1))
 (segment (start 151.0125 97.0375) (end 151.05 97) (width 0.5) (layer "F.Cu") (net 1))
 (segment (start 129.725 100.475) (end 131.095 100.475) (width 0.5) (layer "F.Cu") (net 1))
 (segment (start 134 105.25) (end 134 104) (width 0.5) (layer "F.Cu") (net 1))
 (segment (start 144.26 96) (end 146.75 96) (width 0.5) (layer "F.Cu") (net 1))
 (segment (start 144.05 94.29) (end 144.05 95.79) (width 0.5) (layer "F.Cu") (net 1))
 (segment (start 155 93.75) (end 155 94.9625) (width 0.5) (layer "F.Cu") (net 1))
 (via (at 129.725 100.475) (size 0.8) (drill 0.4) (layers "F.Cu" "B.Cu") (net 1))
 (via (at 129.580713 91.169287) (size 0.8) (drill 0.4) (layers "F.Cu" "B.Cu") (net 1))
 (segment (start 129.75 100.45) (end 129.725 100.475) (width 0.5) (layer "B.Cu") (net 1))
 (segment (start 129.75 91.338574) (end 129.75 100.45) (width 0.5) (layer "B.Cu") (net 1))
 (segment (start 129.580713 91.169287) (end 129.75 91.338574) (width 0.5) (layer "B.Cu") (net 1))
 (segment (start 126 90) (end 123.025 90) (width 0.5) (layer "F.Cu") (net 17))
 (segment (start 145 104.5) (end 145 103.35) (width 0.5) (layer "F.Cu") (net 8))
 (segment (start 142.75 102.75) (end 142.75 104.5) (width 0.5) (layer "F.Cu") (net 8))
 (segment (start 141 101.9625) (end 141.9625 101.9625) (width 0.5) (layer "F.Cu") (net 8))
 (segment (start 142.75 104.5) (end 143 104.75) (width 0.5) (layer "F.Cu") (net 8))
 (segment (start 143 104.75) (end 144.75 104.75) (width 0.5) (layer "F.Cu") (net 8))
 (segment (start 144.75 104.75) (end 145 104.5) (width 0.5) (layer "F.Cu") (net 8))
 (segment (start 141 99) (end 141 101.9625) (width 0.5) (layer "F.Cu") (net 8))
 (segment (start 141.9625 101.9625) (end 142.75 102.75) (width 0.5) (layer "F.Cu") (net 8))
 (segment (start 145 101.705) (end 145.295 102) (width 0.5) (layer "F.Cu") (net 6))
 (segment (start 145.295 102) (end 149 102) (width 0.5) (layer "F.Cu") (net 6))
 (segment (start 145 100.65) (end 145 101.705) (width 0.5) (layer "F.Cu") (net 6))
 (segment (start 140.5 91) (end 144 91) (width 0.5) (layer "F.Cu") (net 4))
 (segment (start 135.9625 96.9625) (end 138 96.9625) (width 0.5) (layer "F.Cu") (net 4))
 (segment (start 152 102) (end 152 100.25) (width 0.5) (layer "F.Cu") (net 4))
 (segment (start 140.9625 96.9625) (end 141 97) (width 0.5) (layer "F.Cu") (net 4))
 (segment (start 141 94) (end 144 91) (width 0.5) (layer "F.Cu") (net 4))
 (segment (start 134.905 95.905) (end 135.9625 96.9625) (width 0.5) (layer "F.Cu") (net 4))
 (segment (start 141 95.25) (end 141 94) (width 0.5) (layer "F.Cu") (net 4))
 (segment (start 141 97) (end 141 95.25) (width 0.5) (layer "F.Cu") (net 4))
 (segment (start 138 96.9625) (end 140.9625 96.9625) (width 0.5) (layer "F.Cu") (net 4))
 (segment (start 134.905 95.525) (end 134.905 95.905) (width 0.5) (layer "F.Cu") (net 4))
 (via (at 141 95.25) (size 0.8) (drill 0.4) (layers "F.Cu" "B.Cu") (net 4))
 (via (at 152 100.25) (size 0.8) (drill 0.4) (layers "F.Cu" "B.Cu") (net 4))
 (segment (start 143.5 100.25) (end 141 97.75) (width 0.5) (layer "B.Cu") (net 4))
 (segment (start 152 100.25) (end 143.5 100.25) (width 0.5) (layer "B.Cu") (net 4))
 (segment (start 141 97.75) (end 141 95.25) (width 0.5) (layer "B.Cu") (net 4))
 (segment (start 135.8 91.95) (end 137.5 91.95) (width 0.5) (layer "F.Cu") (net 3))
 (segment (start 137.5 92.75) (end 138 93.25) (width 0.5) (layer "F.Cu") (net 3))
 (segment (start 138.05 91.95) (end 137.5 91.95) (width 0.5) (layer "F.Cu") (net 3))
 (segment (start 140.05 89.2) (end 139 90.25) (width 0.5) (layer "F.Cu") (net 3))
 (segment (start 137.5 91.95) (end 137.5 92.75) (width 0.5) (layer "F.Cu") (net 3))
 (segment (start 151.9625 94.9625) (end 152 95) (width 0.5) (layer "F.Cu") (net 3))
 (segment (start 149 94.9625) (end 149 93.4) (width 0.5) (layer "F.Cu") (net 3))
 (segment (start 138 93.25) (end 138 94.25) (width 0.5) (layer "F.Cu") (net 3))
 (segment (start 149 93.4) (end 149.7 92.7) (width 0.5) (layer "F.Cu") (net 3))
 (segment (start 149.7 90.1) (end 148.8 89.2) (width 0.5) (layer "F.Cu") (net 3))
 (segment (start 148.8 89.2) (end 140.05 89.2) (width 0.5) (layer "F.Cu") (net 3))
 (segment (start 149 94.9625) (end 151.9625 94.9625) (width 0.5) (layer "F.Cu") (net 3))
 (segment (start 135.35 92.4) (end 135.8 91.95) (width 0.5) (layer "F.Cu") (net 3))
 (segment (start 134 92.4) (end 135.35 92.4) (width 0.5) (layer "F.Cu") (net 3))
 (segment (start 139 90.25) (end 139 91) (width 0.5) (layer "F.Cu") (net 3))
 (segment (start 149.7 92.7) (end 149.7 90.1) (width 0.5) (layer "F.Cu") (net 3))
 (segment (start 139 91) (end 138.05 91.95) (width 0.5) (layer "F.Cu") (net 3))
 (segment (start 145.95 94.29) (end 145.95 93.05) (width 0.5) (layer "F.Cu") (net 16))
 (segment (start 145.95 93.05) (end 148 91) (width 0.5) (layer "F.Cu") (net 16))
 (segment (start 144.05 100.65) (end 144 97.71) (width 0.5) (layer "F.Cu") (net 19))
 (segment (start 145.95 97.71) (end 145.95 100.65) (width 0.5) (layer "F.Cu") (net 21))
 (segment (start 154 102) (end 153.5 102.5) (width 0.5) (layer "F.Cu") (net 5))
 (segment (start 153 104) (end 153.5 103.5) (width 0.5) (layer "F.Cu") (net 5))
 (segment (start 159 100.46) (end 155.54 100.46) (width 0.5) (layer "F.Cu") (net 5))
 (segment (start 152 104) (end 153 104) (width 0.5) (layer "F.Cu") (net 5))
 (segment (start 153.5 102.5) (end 153.5 103.5) (width 0.5) (layer "F.Cu") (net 5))
 (segment (start 155 102) (end 154 102) (width 0.5) (layer "F.Cu") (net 5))
 (segment (start 155 101) (end 155 102) (width 0.5) (layer "F.Cu") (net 5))
 (segment (start 155.54 100.46) (end 155 101) (width 0.5) (layer "F.Cu") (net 5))
 (segment (start 128.75 93.75) (end 128 93) (width 0.5) (layer "F.Cu") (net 11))
 (segment (start 131.143528 93.75) (end 128.75 93.75) (width 0.5) (layer "F.Cu") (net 11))
 (segment (start 132.365 94.971472) (end 131.143528 93.75) (width 0.5) (layer "F.Cu") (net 11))
 (segment (start 132.365 95.525) (end 132.365 94.971472) (width 0.5) (layer "F.Cu") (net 11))
 (segment (start 133.635 94.971472) (end 131.713528 93.05) (width 0.5) (layer "F.Cu") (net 10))
 (segment (start 131.713528 93.05) (end 130.260051 93.05) (width 0.5) (layer "F.Cu") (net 10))
 (segment (start 128 90.789949) (end 128 90) (width 0.5) (layer "F.Cu") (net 10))
 (segment (start 130.260051 93.05) (end 128 90.789949) (width 0.5) (layer "F.Cu") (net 10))
 (segment (start 133.635 95.525) (end 133.635 94.971472) (width 0.5) (layer "F.Cu") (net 10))
 (segment (start 132.365 102.135) (end 132 102.5) (width 0.5) (layer "F.Cu") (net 9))
 (segment (start 132.365 100.475) (end 132.365 102.135) (width 0.5) (layer "F.Cu") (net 9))
 (segment (start 132 102.5) (end 132 104) (width 0.5) (layer "F.Cu") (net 9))
 (segment (start 152.95 97) (end 154.9625 97) (width 0.5) (layer "F.Cu") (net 2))
 (segment (start 155 97.0375) (end 156.2875 97.0375) (width 0.5) (layer "F.Cu") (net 2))
 (segment (start 157 92.25) (end 157 96.325) (width 0.5) (layer "F.Cu") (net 2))
 (segment (start 156.25 91.5) (end 157 92.25) (width 0.5) (layer "F.Cu") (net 2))
 (segment (start 157 96.325) (end 156.2875 97.0375) (width 0.5) (layer "F.Cu") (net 2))
 (segment (start 156.2875 97.0375) (end 157.17 97.92) (width 0.5) (layer "F.Cu") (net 2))
 (segment (start 157.17 97.92) (end 159 97.92) (width 0.5) (layer "F.Cu") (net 2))
 (segment (start 155 91.5) (end 156.25 91.5) (width 0.5) (layer "F.Cu") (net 2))
 (segment (start 154.9625 97) (end 155 97.0375) (width 0.5) (layer "F.Cu") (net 2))
 (segment (start 157 89.25) (end 159 91.25) (width 0.5) (layer "F.Cu") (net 22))
 (segment (start 151 89.25) (end 157 89.25) (width 0.5) (layer "F.Cu") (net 22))
 (segment (start 151.2 92.45) (end 150.5 91.75) (width 0.5) (layer "F.Cu") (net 22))
 (segment (start 152 92.45) (end 151.2 92.45) (width 0.5) (layer "F.Cu") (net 22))
 (segment (start 150.5 91.75) (end 150.5 89.75) (width 0.5) (layer "F.Cu") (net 22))
 (segment (start 150.5 89.75) (end 151 89.25) (width 0.5) (layer "F.Cu") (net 22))
 (segment (start 159 91.25) (end 159 95.38) (width 0.5) (layer "F.Cu") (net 22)))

